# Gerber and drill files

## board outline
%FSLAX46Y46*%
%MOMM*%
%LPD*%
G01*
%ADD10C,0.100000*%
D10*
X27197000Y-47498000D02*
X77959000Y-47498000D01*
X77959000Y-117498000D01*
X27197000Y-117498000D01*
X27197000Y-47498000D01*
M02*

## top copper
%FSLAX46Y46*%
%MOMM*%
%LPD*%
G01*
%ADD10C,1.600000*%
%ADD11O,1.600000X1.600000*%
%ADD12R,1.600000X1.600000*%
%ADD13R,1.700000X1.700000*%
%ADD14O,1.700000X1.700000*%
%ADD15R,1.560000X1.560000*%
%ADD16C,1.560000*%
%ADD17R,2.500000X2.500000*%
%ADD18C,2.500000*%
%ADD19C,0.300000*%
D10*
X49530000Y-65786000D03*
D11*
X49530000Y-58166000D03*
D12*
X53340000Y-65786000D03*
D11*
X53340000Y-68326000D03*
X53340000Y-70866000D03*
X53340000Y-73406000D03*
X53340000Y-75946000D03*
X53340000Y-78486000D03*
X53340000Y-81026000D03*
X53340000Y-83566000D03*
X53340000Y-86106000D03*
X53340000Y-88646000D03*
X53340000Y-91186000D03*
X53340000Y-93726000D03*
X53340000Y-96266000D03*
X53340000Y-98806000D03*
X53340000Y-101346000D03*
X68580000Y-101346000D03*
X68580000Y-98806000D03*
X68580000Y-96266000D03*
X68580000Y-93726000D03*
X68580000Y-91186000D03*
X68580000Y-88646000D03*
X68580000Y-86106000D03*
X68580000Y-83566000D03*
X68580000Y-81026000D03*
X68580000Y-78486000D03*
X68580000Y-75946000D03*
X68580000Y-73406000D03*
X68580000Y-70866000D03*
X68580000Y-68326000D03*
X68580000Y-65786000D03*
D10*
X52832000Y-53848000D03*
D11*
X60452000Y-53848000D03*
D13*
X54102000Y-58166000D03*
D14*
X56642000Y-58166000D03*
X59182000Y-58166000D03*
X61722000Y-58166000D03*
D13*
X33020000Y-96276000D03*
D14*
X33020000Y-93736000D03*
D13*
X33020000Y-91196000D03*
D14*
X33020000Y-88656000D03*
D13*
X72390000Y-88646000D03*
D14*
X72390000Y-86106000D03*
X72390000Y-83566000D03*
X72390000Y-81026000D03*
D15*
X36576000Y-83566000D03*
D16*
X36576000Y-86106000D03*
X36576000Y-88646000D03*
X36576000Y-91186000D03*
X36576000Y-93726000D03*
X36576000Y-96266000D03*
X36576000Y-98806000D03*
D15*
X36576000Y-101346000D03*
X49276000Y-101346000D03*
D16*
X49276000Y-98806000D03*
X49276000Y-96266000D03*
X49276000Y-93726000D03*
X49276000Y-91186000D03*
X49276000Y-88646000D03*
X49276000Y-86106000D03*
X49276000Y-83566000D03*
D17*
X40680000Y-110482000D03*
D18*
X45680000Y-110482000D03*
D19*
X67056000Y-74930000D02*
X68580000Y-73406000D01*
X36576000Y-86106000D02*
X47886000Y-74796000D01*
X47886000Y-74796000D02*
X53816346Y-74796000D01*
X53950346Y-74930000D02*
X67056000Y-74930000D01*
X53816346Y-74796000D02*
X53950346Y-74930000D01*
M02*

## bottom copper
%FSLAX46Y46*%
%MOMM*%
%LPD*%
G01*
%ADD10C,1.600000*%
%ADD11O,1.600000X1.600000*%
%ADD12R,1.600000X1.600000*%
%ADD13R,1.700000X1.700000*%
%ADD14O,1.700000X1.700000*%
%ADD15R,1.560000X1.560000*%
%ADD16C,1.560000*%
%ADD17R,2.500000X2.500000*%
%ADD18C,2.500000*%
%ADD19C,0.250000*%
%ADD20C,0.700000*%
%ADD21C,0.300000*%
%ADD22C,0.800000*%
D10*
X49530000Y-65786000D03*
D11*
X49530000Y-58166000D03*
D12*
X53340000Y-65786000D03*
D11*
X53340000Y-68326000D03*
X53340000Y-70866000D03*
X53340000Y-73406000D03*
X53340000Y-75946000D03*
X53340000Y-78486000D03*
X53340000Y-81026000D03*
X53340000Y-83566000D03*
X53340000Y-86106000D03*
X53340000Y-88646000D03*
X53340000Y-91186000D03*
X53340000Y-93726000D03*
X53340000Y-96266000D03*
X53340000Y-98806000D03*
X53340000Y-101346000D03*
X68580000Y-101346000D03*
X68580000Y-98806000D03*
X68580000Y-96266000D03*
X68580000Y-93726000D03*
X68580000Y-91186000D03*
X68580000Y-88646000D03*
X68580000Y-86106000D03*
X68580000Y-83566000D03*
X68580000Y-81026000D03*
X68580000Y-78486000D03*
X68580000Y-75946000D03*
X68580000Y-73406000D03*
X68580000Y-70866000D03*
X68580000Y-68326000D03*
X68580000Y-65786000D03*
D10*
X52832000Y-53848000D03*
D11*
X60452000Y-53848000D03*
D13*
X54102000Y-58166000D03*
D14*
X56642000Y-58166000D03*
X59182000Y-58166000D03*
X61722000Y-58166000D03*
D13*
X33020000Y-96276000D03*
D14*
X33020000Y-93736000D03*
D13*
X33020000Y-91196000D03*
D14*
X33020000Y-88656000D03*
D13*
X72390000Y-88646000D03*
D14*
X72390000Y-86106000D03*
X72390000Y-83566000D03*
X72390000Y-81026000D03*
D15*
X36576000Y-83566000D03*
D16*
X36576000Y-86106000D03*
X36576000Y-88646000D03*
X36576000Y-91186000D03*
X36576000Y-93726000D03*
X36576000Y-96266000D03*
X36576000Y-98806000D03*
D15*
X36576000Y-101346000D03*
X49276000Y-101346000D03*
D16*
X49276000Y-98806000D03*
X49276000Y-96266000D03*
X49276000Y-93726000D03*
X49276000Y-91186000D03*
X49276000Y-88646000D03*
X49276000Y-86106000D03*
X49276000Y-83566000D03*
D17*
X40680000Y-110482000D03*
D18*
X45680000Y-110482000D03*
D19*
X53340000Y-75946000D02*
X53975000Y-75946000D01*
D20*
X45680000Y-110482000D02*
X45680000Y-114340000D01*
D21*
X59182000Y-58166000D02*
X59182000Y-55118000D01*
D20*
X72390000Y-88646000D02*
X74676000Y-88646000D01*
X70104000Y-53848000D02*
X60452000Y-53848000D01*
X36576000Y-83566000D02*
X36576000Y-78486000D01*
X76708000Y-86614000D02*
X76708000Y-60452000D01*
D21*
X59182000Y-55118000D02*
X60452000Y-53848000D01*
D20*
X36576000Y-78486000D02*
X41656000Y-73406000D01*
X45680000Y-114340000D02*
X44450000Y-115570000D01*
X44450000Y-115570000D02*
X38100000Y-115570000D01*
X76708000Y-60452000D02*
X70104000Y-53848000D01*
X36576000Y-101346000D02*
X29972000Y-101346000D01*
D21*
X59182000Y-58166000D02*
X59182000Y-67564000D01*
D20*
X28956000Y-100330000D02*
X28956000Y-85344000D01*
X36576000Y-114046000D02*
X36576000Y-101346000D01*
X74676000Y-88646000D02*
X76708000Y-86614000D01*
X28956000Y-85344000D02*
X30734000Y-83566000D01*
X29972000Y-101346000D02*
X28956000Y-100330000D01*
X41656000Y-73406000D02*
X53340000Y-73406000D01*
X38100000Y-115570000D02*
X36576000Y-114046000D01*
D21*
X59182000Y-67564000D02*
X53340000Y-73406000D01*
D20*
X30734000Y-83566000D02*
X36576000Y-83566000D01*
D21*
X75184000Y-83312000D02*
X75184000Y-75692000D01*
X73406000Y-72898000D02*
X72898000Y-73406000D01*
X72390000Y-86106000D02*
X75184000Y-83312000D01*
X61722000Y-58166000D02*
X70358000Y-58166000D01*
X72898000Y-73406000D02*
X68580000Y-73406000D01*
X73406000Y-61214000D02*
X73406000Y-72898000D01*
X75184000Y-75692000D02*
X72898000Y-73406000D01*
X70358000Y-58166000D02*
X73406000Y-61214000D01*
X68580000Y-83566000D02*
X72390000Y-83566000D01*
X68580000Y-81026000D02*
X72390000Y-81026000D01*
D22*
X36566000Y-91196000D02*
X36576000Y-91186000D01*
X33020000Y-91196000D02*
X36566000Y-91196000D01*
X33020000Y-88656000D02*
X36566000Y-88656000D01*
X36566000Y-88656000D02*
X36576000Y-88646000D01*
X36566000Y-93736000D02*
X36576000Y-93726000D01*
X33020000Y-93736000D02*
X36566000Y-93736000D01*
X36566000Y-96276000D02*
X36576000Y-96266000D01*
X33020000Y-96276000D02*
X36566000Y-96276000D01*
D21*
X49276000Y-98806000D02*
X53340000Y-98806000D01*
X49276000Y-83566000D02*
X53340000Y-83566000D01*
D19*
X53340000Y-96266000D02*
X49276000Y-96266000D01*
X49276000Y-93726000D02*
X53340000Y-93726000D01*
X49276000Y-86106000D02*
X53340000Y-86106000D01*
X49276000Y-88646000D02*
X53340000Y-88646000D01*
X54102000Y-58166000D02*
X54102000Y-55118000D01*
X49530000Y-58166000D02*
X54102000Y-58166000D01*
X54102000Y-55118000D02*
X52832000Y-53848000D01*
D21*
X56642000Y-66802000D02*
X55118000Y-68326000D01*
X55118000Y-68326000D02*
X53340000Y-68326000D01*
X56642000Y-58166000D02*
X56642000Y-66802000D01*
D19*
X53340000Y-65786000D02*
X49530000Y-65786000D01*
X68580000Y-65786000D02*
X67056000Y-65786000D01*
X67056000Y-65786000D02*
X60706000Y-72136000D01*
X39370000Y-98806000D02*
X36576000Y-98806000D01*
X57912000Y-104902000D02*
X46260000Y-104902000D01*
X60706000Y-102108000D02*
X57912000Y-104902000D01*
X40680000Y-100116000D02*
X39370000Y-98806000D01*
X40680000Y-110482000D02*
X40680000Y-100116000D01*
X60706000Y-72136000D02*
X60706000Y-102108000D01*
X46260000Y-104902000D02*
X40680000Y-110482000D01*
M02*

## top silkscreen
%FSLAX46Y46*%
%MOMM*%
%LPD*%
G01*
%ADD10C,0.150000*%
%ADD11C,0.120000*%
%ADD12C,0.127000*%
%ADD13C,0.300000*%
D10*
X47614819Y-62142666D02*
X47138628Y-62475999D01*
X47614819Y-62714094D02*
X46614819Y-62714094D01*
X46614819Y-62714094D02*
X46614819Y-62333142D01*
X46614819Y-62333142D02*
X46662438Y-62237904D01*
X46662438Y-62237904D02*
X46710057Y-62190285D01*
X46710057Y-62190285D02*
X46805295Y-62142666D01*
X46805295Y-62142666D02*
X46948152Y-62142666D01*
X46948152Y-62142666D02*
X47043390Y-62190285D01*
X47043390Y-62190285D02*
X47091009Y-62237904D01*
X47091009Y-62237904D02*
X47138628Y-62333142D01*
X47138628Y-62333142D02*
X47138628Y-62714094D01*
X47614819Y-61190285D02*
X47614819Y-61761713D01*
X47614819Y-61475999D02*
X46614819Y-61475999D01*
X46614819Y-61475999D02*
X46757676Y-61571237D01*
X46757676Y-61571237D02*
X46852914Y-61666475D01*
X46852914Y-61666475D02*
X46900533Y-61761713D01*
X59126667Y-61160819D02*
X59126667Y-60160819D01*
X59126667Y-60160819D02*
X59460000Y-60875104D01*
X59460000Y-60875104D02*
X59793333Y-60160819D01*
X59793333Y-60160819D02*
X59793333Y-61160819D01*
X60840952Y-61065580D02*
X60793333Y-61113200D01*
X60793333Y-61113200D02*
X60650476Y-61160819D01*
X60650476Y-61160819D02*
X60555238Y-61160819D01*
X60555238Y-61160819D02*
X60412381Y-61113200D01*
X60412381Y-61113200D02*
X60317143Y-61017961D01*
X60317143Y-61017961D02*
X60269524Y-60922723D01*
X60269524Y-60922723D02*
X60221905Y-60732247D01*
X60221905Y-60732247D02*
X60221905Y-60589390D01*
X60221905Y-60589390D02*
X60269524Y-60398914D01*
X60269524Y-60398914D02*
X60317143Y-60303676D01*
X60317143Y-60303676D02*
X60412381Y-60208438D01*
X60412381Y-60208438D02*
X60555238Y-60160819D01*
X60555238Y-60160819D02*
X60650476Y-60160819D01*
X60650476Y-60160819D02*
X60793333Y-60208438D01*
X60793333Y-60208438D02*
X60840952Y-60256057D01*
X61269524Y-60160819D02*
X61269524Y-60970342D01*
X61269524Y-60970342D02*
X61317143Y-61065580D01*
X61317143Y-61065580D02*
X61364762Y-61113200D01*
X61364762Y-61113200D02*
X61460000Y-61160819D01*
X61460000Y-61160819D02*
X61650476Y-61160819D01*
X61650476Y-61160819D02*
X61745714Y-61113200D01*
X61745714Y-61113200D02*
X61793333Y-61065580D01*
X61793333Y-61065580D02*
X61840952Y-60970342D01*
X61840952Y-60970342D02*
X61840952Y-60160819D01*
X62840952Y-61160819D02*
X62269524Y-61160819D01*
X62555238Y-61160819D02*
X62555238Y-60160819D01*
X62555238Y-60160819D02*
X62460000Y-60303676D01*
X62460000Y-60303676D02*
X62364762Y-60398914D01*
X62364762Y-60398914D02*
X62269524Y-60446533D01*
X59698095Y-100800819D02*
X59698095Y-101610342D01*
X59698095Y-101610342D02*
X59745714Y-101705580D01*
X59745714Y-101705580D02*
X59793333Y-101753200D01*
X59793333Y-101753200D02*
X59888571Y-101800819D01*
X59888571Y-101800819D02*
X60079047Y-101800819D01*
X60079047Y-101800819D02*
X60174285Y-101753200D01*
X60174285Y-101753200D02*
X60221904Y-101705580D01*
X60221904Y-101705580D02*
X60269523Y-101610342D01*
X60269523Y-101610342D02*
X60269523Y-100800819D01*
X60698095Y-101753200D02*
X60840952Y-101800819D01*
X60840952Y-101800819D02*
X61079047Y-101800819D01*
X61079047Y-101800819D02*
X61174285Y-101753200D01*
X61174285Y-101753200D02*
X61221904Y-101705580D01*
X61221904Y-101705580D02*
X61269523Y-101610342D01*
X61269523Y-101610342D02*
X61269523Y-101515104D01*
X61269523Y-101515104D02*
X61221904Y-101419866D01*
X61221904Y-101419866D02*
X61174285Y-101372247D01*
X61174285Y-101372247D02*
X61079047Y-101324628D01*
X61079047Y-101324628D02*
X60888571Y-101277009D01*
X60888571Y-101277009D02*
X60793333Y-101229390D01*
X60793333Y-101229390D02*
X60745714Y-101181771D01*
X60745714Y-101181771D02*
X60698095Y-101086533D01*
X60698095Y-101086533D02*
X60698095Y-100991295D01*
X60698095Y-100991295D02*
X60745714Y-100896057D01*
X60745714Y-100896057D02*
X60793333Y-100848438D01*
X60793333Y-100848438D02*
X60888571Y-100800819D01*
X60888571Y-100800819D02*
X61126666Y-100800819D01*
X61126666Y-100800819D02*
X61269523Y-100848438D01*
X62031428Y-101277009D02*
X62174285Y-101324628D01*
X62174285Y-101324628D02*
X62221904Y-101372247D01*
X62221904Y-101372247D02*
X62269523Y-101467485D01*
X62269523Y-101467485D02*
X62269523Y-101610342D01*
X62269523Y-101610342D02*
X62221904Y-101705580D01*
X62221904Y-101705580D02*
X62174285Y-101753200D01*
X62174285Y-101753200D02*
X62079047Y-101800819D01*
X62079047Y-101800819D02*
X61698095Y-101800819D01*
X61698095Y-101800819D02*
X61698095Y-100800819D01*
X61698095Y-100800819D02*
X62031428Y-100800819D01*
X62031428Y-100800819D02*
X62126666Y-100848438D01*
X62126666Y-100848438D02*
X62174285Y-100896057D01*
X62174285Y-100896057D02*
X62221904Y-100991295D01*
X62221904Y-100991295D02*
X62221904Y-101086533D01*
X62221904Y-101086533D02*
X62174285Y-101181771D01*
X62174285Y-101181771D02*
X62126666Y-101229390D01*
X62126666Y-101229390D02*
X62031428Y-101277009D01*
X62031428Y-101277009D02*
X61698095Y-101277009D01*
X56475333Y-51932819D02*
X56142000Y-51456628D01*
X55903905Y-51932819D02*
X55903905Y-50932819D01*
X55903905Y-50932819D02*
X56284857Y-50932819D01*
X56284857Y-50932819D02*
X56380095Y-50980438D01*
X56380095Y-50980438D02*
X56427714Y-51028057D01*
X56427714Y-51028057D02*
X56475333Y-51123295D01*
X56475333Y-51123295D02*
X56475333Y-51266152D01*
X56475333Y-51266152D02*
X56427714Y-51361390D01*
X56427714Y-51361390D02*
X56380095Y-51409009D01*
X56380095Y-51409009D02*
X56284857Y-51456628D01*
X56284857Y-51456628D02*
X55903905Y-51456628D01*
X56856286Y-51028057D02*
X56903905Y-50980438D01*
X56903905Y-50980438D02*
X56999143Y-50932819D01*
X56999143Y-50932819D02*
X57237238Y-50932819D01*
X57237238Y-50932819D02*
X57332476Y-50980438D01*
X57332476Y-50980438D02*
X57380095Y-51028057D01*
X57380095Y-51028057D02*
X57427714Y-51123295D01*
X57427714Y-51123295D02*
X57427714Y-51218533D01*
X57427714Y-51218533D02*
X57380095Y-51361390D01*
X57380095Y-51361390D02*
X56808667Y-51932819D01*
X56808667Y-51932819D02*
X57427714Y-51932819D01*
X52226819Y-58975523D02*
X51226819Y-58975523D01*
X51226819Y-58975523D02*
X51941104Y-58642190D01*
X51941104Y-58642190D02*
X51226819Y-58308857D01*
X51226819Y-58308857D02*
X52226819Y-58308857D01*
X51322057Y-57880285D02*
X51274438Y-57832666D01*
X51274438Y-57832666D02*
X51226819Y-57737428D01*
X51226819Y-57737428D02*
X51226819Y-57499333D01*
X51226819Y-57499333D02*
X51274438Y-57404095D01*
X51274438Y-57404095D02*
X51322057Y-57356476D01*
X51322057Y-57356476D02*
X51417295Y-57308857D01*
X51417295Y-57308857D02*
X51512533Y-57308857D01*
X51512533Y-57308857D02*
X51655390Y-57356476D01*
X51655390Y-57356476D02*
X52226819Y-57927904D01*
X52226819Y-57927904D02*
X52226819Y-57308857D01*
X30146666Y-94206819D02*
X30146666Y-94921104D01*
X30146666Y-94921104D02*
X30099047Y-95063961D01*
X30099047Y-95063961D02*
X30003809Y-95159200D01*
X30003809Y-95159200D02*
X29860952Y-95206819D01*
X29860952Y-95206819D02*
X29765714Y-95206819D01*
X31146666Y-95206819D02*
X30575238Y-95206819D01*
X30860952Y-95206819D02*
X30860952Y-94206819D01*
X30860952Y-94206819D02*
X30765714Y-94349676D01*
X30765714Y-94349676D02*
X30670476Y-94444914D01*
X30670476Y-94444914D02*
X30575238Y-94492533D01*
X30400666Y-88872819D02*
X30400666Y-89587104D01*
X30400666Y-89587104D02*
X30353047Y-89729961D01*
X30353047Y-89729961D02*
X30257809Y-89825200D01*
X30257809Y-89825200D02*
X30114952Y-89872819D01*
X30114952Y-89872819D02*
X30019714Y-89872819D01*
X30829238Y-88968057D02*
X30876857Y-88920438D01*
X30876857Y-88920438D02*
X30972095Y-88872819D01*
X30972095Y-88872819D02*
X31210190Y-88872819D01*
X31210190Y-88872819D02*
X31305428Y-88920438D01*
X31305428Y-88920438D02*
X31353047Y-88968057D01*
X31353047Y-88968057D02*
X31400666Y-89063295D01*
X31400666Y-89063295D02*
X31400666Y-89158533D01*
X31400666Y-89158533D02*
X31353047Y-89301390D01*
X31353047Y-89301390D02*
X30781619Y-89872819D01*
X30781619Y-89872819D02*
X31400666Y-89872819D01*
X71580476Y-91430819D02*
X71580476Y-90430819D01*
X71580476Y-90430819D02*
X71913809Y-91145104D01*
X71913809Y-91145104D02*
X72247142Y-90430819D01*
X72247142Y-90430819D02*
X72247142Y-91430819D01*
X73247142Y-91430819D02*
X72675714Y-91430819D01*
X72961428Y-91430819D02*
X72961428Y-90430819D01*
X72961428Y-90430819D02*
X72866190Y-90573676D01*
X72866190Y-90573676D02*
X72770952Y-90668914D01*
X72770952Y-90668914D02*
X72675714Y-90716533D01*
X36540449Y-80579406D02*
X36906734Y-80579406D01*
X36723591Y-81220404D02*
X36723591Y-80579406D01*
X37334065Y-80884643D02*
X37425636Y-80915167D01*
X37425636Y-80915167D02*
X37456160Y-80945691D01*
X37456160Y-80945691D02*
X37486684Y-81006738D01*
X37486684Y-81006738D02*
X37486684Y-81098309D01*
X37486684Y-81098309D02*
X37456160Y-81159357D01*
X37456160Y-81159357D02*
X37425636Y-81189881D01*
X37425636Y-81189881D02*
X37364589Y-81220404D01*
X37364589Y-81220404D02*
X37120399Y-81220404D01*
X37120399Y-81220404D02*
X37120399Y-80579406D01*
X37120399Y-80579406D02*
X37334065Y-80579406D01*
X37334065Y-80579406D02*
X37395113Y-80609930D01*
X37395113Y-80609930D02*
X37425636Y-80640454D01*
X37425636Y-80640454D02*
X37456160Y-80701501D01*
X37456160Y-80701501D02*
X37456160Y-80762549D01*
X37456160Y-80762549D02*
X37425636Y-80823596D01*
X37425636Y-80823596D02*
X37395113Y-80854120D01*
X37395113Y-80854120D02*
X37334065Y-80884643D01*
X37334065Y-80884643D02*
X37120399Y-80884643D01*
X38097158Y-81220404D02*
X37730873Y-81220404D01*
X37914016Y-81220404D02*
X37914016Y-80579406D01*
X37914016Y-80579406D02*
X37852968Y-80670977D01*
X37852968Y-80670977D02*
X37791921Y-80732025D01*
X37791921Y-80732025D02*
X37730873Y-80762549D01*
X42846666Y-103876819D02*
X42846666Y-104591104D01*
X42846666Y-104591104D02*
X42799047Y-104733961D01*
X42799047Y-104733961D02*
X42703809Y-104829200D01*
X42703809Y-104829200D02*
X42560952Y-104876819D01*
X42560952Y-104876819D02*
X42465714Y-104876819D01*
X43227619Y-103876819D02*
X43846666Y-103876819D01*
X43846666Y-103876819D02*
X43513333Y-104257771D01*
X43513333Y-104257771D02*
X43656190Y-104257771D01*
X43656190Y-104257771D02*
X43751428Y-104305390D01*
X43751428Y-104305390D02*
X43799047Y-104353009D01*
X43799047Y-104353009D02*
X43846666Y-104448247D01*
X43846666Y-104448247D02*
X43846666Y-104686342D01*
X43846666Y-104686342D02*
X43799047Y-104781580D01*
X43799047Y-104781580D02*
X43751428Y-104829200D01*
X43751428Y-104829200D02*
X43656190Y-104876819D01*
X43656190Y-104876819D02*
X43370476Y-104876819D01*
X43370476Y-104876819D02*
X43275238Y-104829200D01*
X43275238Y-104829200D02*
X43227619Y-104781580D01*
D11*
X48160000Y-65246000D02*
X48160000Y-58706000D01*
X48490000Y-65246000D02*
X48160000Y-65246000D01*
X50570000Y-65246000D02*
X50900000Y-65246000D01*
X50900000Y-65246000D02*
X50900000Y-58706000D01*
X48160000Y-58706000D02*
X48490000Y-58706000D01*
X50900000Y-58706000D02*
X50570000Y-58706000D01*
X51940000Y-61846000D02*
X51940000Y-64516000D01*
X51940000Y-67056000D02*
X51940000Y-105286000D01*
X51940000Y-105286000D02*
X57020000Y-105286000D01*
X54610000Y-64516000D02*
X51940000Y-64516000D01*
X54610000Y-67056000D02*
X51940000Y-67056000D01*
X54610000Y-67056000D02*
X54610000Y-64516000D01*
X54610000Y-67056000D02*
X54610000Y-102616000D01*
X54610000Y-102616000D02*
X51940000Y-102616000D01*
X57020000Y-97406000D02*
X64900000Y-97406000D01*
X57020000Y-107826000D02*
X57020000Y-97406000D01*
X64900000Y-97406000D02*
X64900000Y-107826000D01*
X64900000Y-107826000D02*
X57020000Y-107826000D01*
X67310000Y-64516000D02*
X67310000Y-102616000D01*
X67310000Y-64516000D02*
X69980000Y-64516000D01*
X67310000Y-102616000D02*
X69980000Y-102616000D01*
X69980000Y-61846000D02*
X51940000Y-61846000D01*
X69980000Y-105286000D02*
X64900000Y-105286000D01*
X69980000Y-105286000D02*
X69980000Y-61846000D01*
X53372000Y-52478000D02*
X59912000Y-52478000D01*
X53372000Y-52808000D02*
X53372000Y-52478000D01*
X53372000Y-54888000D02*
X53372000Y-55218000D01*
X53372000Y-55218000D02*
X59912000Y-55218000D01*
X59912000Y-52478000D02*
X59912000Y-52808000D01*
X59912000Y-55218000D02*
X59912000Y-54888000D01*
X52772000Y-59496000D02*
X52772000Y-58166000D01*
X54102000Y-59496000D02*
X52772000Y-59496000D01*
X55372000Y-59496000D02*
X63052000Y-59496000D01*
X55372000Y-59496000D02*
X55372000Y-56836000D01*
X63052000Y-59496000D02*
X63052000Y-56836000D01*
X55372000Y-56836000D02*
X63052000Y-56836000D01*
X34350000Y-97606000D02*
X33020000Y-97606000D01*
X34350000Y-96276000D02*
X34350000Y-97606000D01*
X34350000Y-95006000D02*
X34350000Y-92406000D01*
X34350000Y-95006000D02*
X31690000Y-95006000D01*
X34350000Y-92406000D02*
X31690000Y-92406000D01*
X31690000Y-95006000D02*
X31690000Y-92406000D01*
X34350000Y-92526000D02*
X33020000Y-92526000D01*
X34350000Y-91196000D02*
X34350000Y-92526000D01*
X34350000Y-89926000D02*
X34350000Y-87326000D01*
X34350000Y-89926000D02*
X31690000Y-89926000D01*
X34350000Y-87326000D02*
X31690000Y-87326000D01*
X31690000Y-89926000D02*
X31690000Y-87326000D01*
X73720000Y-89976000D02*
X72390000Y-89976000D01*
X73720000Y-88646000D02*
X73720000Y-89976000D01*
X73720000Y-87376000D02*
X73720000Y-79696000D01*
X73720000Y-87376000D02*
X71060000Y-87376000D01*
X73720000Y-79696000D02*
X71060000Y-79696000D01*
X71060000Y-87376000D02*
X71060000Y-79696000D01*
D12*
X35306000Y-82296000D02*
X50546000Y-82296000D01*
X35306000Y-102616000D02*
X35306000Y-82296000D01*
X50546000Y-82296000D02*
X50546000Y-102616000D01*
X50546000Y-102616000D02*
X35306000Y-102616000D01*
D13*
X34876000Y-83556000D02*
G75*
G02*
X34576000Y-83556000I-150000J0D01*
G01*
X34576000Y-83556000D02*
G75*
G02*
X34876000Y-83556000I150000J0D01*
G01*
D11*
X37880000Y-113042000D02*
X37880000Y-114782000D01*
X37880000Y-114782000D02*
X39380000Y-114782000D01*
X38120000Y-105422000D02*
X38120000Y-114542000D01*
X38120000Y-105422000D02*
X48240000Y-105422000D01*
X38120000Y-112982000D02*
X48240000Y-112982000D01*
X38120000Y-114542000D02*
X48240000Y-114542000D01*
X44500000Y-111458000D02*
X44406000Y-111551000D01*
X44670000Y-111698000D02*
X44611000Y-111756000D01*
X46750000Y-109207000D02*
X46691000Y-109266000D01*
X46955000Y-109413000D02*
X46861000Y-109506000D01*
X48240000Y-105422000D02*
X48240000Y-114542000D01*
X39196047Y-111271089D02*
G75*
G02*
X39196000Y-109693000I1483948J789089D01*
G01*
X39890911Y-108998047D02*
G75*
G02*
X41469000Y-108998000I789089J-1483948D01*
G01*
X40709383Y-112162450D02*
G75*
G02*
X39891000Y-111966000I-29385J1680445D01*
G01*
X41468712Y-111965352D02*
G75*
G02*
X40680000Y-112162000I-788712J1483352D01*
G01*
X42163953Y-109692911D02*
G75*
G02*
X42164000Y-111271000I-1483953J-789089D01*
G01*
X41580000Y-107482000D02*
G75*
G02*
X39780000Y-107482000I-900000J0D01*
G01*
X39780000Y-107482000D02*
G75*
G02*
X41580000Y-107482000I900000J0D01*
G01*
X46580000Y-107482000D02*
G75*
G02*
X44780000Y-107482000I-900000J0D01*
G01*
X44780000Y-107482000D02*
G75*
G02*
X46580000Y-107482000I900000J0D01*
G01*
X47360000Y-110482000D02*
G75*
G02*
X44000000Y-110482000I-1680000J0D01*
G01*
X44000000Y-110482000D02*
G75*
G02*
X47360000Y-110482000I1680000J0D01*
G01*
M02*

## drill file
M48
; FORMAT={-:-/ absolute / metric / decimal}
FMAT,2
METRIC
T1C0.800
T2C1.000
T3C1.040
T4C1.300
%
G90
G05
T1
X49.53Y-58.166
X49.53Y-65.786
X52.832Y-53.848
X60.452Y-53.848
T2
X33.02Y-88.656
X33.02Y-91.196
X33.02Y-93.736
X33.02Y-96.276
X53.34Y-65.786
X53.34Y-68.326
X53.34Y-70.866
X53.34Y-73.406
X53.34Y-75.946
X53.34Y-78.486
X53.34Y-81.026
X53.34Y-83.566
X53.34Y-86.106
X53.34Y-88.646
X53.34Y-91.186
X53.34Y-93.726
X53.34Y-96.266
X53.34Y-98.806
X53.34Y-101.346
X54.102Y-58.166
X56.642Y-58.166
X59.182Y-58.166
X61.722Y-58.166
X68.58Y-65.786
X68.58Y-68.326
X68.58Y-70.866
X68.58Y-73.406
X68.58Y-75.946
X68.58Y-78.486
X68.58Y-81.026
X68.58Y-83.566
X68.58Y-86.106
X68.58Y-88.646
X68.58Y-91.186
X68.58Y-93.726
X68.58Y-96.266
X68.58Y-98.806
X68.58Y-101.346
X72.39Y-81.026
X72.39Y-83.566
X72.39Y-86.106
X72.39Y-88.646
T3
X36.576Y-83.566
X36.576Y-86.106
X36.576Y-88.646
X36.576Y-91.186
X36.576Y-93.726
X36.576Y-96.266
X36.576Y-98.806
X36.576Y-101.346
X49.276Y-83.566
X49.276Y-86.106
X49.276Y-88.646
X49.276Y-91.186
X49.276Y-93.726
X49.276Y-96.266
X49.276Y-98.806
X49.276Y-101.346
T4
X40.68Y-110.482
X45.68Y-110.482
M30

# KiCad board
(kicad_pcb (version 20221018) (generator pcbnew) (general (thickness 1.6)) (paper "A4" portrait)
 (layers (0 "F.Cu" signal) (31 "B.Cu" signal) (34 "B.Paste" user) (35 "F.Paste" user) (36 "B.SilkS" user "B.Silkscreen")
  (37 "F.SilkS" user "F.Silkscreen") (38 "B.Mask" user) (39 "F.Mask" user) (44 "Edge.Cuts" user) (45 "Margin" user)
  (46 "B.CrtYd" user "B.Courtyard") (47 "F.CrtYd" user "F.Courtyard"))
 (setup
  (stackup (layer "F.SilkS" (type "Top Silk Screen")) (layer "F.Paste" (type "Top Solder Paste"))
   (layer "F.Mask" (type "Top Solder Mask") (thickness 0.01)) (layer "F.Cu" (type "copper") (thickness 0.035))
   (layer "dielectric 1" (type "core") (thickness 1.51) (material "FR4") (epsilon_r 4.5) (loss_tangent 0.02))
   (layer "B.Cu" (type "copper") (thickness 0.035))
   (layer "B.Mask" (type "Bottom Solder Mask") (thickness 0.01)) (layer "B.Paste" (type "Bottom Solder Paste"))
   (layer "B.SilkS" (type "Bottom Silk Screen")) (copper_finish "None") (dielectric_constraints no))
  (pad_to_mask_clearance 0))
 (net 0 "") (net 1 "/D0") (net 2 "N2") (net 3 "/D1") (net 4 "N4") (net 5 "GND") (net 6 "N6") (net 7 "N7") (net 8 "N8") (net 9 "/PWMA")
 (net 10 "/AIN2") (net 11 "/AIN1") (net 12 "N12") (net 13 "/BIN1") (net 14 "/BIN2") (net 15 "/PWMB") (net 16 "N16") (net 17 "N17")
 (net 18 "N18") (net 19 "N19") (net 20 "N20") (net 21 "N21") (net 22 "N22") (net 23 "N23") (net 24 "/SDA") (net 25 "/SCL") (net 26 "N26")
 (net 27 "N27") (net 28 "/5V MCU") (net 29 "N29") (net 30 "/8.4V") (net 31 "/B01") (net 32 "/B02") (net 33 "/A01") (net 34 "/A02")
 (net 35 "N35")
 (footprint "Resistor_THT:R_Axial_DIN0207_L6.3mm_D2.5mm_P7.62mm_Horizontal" (layer "F.Cu") (at 49.53 65.786 90)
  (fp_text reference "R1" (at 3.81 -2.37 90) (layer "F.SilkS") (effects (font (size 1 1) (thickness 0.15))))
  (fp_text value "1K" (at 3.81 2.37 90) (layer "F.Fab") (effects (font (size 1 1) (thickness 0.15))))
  (fp_line (start 0.54 -1.37) (end 7.08 -1.37) (stroke (width 0.12) (type solid)) (layer "F.SilkS"))
  (fp_line (start 0.54 -1.04) (end 0.54 -1.37) (stroke (width 0.12) (type solid)) (layer "F.SilkS"))
  (fp_line (start 0.54 1.04) (end 0.54 1.37) (stroke (width 0.12) (type solid)) (layer "F.SilkS"))
  (fp_line (start 0.54 1.37) (end 7.08 1.37) (stroke (width 0.12) (type solid)) (layer "F.SilkS"))
  (fp_line (start 7.08 -1.37) (end 7.08 -1.04) (stroke (width 0.12) (type solid)) (layer "F.SilkS"))
  (fp_line (start 7.08 1.37) (end 7.08 1.04) (stroke (width 0.12) (type solid)) (layer "F.SilkS"))
  (pad "1" thru_hole circle (at 0 0 90) (size 1.6 1.6) (drill 0.8) (layers "*.Cu" "*.Mask") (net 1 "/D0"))
  (pad "2" thru_hole oval (at 7.62 0 90) (size 1.6 1.6) (drill 0.8) (layers "*.Cu" "*.Mask") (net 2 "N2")))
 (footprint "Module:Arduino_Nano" (layer "F.Cu") (at 53.34 65.786)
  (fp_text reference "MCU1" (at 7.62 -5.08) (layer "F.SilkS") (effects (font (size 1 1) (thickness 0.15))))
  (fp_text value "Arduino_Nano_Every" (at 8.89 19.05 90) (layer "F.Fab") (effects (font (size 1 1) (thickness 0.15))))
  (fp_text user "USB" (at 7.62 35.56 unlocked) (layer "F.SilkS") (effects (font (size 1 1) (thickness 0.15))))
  (fp_line (start -1.4 -3.94) (end -1.4 -1.27) (stroke (width 0.12) (type solid)) (layer "F.SilkS"))
  (fp_line (start -1.4 1.27) (end -1.4 39.5) (stroke (width 0.12) (type solid)) (layer "F.SilkS"))
  (fp_line (start -1.4 39.5) (end 3.68 39.5) (stroke (width 0.12) (type solid)) (layer "F.SilkS"))
  (fp_line (start 1.27 -1.27) (end -1.4 -1.27) (stroke (width 0.12) (type solid)) (layer "F.SilkS"))
  (fp_line (start 1.27 1.27) (end -1.4 1.27) (stroke (width 0.12) (type solid)) (layer "F.SilkS"))
  (fp_line (start 1.27 1.27) (end 1.27 -1.27) (stroke (width 0.12) (type solid)) (layer "F.SilkS"))
  (fp_line (start 1.27 1.27) (end 1.27 36.83) (stroke (width 0.12) (type solid)) (layer "F.SilkS"))
  (fp_line (start 1.27 36.83) (end -1.4 36.83) (stroke (width 0.12) (type solid)) (layer "F.SilkS"))
  (fp_line (start 3.68 31.62) (end 11.56 31.62) (stroke (width 0.12) (type solid)) (layer "F.SilkS"))
  (fp_line (start 3.68 42.04) (end 3.68 31.62) (stroke (width 0.12) (type solid)) (layer "F.SilkS"))
  (fp_line (start 11.56 31.62) (end 11.56 42.04) (stroke (width 0.12) (type solid)) (layer "F.SilkS"))
  (fp_line (start 11.56 42.04) (end 3.68 42.04) (stroke (width 0.12) (type solid)) (layer "F.SilkS"))
  (fp_line (start 13.97 -1.27) (end 13.97 36.83) (stroke (width 0.12) (type solid)) (layer "F.SilkS"))
  (fp_line (start 13.97 -1.27) (end 16.64 -1.27) (stroke (width 0.12) (type solid)) (layer "F.SilkS"))
  (fp_line (start 13.97 36.83) (end 16.64 36.83) (stroke (width 0.12) (type solid)) (layer "F.SilkS"))
  (fp_line (start 16.64 -3.94) (end -1.4 -3.94) (stroke (width 0.12) (type solid)) (layer "F.SilkS"))
  (fp_line (start 16.64 39.5) (end 11.56 39.5) (stroke (width 0.12) (type solid)) (layer "F.SilkS"))
  (fp_line (start 16.64 39.5) (end 16.64 -3.94) (stroke (width 0.12) (type solid)) (layer "F.SilkS"))
  (pad "1" thru_hole rect (at 0 0) (size 1.6 1.6) (drill 1) (layers "*.Cu" "*.Mask") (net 1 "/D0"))
  (pad "2" thru_hole oval (at 0 2.54) (size 1.6 1.6) (drill 1) (layers "*.Cu" "*.Mask") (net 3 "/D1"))
  (pad "3" thru_hole oval (at 0 5.08) (size 1.6 1.6) (drill 1) (layers "*.Cu" "*.Mask") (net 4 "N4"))
  (pad "4" thru_hole oval (at 0 7.62) (size 1.6 1.6) (drill 1) (layers "*.Cu" "*.Mask") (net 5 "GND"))
  (pad "5" thru_hole oval (at 0 10.16) (size 1.6 1.6) (drill 1) (layers "*.Cu" "*.Mask") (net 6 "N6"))
  (pad "6" thru_hole oval (at 0 12.7) (size 1.6 1.6) (drill 1) (layers "*.Cu" "*.Mask") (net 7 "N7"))
  (pad "7" thru_hole oval (at 0 15.24) (size 1.6 1.6) (drill 1) (layers "*.Cu" "*.Mask") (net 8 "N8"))
  (pad "8" thru_hole oval (at 0 17.78) (size 1.6 1.6) (drill 1) (layers "*.Cu" "*.Mask") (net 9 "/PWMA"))
  (pad "9" thru_hole oval (at 0 20.32) (size 1.6 1.6) (drill 1) (layers "*.Cu" "*.Mask") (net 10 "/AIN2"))
  (pad "10" thru_hole oval (at 0 22.86) (size 1.6 1.6) (drill 1) (layers "*.Cu" "*.Mask") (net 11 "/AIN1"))
  (pad "11" thru_hole oval (at 0 25.4) (size 1.6 1.6) (drill 1) (layers "*.Cu" "*.Mask") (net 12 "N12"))
  (pad "12" thru_hole oval (at 0 27.94) (size 1.6 1.6) (drill 1) (layers "*.Cu" "*.Mask") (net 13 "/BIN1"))
  (pad "13" thru_hole oval (at 0 30.48) (size 1.6 1.6) (drill 1) (layers "*.Cu" "*.Mask") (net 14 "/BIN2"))
  (pad "14" thru_hole oval (at 0 33.02) (size 1.6 1.6) (drill 1) (layers "*.Cu" "*.Mask") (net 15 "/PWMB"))
  (pad "15" thru_hole oval (at 0 35.56) (size 1.6 1.6) (drill 1) (layers "*.Cu" "*.Mask") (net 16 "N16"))
  (pad "16" thru_hole oval (at 15.24 35.56) (size 1.6 1.6) (drill 1) (layers "*.Cu" "*.Mask") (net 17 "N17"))
  (pad "17" thru_hole oval (at 15.24 33.02) (size 1.6 1.6) (drill 1) (layers "*.Cu" "*.Mask") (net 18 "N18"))
  (pad "18" thru_hole oval (at 15.24 30.48) (size 1.6 1.6) (drill 1) (layers "*.Cu" "*.Mask") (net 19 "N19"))
  (pad "19" thru_hole oval (at 15.24 27.94) (size 1.6 1.6) (drill 1) (layers "*.Cu" "*.Mask") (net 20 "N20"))
  (pad "20" thru_hole oval (at 15.24 25.4) (size 1.6 1.6) (drill 1) (layers "*.Cu" "*.Mask") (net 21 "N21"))
  (pad "21" thru_hole oval (at 15.24 22.86) (size 1.6 1.6) (drill 1) (layers "*.Cu" "*.Mask") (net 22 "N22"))
  (pad "22" thru_hole oval (at 15.24 20.32) (size 1.6 1.6) (drill 1) (layers "*.Cu" "*.Mask") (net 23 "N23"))
  (pad "23" thru_hole oval (at 15.24 17.78) (size 1.6 1.6) (drill 1) (layers "*.Cu" "*.Mask") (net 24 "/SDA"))
  (pad "24" thru_hole oval (at 15.24 15.24) (size 1.6 1.6) (drill 1) (layers "*.Cu" "*.Mask") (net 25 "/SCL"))
  (pad "25" thru_hole oval (at 15.24 12.7) (size 1.6 1.6) (drill 1) (layers "*.Cu" "*.Mask") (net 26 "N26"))
  (pad "26" thru_hole oval (at 15.24 10.16) (size 1.6 1.6) (drill 1) (layers "*.Cu" "*.Mask") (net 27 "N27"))
  (pad "27" thru_hole oval (at 15.24 7.62) (size 1.6 1.6) (drill 1) (layers "*.Cu" "*.Mask") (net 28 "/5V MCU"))
  (pad "28" thru_hole oval (at 15.24 5.08) (size 1.6 1.6) (drill 1) (layers "*.Cu" "*.Mask") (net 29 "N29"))
  (pad "29" thru_hole oval (at 15.24 2.54) (size 1.6 1.6) (drill 1) (layers "*.Cu" "*.Mask") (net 5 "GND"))
  (pad "30" thru_hole oval (at 15.24 0) (size 1.6 1.6) (drill 1) (layers "*.Cu" "*.Mask") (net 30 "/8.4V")))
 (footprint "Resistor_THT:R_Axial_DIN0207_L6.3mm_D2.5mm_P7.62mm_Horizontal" (layer "F.Cu") (at 52.832 53.848)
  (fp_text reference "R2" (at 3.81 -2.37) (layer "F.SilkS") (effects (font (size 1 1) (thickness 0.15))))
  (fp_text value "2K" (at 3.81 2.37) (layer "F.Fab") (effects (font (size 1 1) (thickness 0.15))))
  (fp_line (start 0.54 -1.37) (end 7.08 -1.37) (stroke (width 0.12) (type solid)) (layer "F.SilkS"))
  (fp_line (start 0.54 -1.04) (end 0.54 -1.37) (stroke (width 0.12) (type solid)) (layer "F.SilkS"))
  (fp_line (start 0.54 1.04) (end 0.54 1.37) (stroke (width 0.12) (type solid)) (layer "F.SilkS"))
  (fp_line (start 0.54 1.37) (end 7.08 1.37) (stroke (width 0.12) (type solid)) (layer "F.SilkS"))
  (fp_line (start 7.08 -1.37) (end 7.08 -1.04) (stroke (width 0.12) (type solid)) (layer "F.SilkS"))
  (fp_line (start 7.08 1.37) (end 7.08 1.04) (stroke (width 0.12) (type solid)) (layer "F.SilkS"))
  (pad "1" thru_hole circle (at 0 0) (size 1.6 1.6) (drill 0.8) (layers "*.Cu" "*.Mask") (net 2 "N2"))
  (pad "2" thru_hole oval (at 7.62 0) (size 1.6 1.6) (drill 0.8) (layers "*.Cu" "*.Mask") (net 5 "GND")))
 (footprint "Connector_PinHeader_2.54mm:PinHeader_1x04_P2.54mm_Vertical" (layer "F.Cu") (at 54.102 58.166 90)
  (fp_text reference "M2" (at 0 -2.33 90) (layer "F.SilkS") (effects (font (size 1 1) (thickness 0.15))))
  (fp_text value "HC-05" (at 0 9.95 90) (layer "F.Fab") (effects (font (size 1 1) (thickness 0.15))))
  (fp_line (start -1.33 -1.33) (end 0 -1.33) (stroke (width 0.12) (type solid)) (layer "F.SilkS"))
  (fp_line (start -1.33 0) (end -1.33 -1.33) (stroke (width 0.12) (type solid)) (layer "F.SilkS"))
  (fp_line (start -1.33 1.27) (end -1.33 8.95) (stroke (width 0.12) (type solid)) (layer "F.SilkS"))
  (fp_line (start -1.33 1.27) (end 1.33 1.27) (stroke (width 0.12) (type solid)) (layer "F.SilkS"))
  (fp_line (start -1.33 8.95) (end 1.33 8.95) (stroke (width 0.12) (type solid)) (layer "F.SilkS"))
  (fp_line (start 1.33 1.27) (end 1.33 8.95) (stroke (width 0.12) (type solid)) (layer "F.SilkS"))
  (pad "1" thru_hole rect (at 0 0 90) (size 1.7 1.7) (drill 1) (layers "*.Cu" "*.Mask") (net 2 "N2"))
  (pad "2" thru_hole oval (at 0 2.54 90) (size 1.7 1.7) (drill 1) (layers "*.Cu" "*.Mask") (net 3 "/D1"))
  (pad "3" thru_hole oval (at 0 5.08 90) (size 1.7 1.7) (drill 1) (layers "*.Cu" "*.Mask") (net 5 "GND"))
  (pad "4" thru_hole oval (at 0 7.62 90) (size 1.7 1.7) (drill 1) (layers "*.Cu" "*.Mask") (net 28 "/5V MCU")))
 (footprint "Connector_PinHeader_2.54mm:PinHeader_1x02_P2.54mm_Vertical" (layer "F.Cu") (at 33.02 96.276 180)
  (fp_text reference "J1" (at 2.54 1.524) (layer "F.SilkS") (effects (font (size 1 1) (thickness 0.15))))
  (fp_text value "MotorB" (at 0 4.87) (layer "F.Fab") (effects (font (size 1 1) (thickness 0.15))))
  (fp_line (start -1.33 -1.33) (end 0 -1.33) (stroke (width 0.12) (type solid)) (layer "F.SilkS"))
  (fp_line (start -1.33 0) (end -1.33 -1.33) (stroke (width 0.12) (type solid)) (layer "F.SilkS"))
  (fp_line (start -1.33 1.27) (end -1.33 3.87) (stroke (width 0.12) (type solid)) (layer "F.SilkS"))
  (fp_line (start -1.33 1.27) (end 1.33 1.27) (stroke (width 0.12) (type solid)) (layer "F.SilkS"))
  (fp_line (start -1.33 3.87) (end 1.33 3.87) (stroke (width 0.12) (type solid)) (layer "F.SilkS"))
  (fp_line (start 1.33 1.27) (end 1.33 3.87) (stroke (width 0.12) (type solid)) (layer "F.SilkS"))
  (pad "1" thru_hole rect (at 0 0 180) (size 1.7 1.7) (drill 1) (layers "*.Cu" "*.Mask") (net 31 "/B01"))
  (pad "2" thru_hole oval (at 0 2.54 180) (size 1.7 1.7) (drill 1) (layers "*.Cu" "*.Mask") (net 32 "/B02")))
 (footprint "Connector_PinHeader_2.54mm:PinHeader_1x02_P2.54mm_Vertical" (layer "F.Cu") (at 33.02 91.196 180)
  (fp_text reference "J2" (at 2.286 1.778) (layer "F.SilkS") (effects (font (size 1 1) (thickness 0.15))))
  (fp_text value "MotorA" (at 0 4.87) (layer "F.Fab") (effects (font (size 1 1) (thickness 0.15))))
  (fp_line (start -1.33 -1.33) (end 0 -1.33) (stroke (width 0.12) (type solid)) (layer "F.SilkS"))
  (fp_line (start -1.33 0) (end -1.33 -1.33) (stroke (width 0.12) (type solid)) (layer "F.SilkS"))
  (fp_line (start -1.33 1.27) (end -1.33 3.87) (stroke (width 0.12) (type solid)) (layer "F.SilkS"))
  (fp_line (start -1.33 1.27) (end 1.33 1.27) (stroke (width 0.12) (type solid)) (layer "F.SilkS"))
  (fp_line (start -1.33 3.87) (end 1.33 3.87) (stroke (width 0.12) (type solid)) (layer "F.SilkS"))
  (fp_line (start 1.33 1.27) (end 1.33 3.87) (stroke (width 0.12) (type solid)) (layer "F.SilkS"))
  (pad "1" thru_hole rect (at 0 0 180) (size 1.7 1.7) (drill 1) (layers "*.Cu" "*.Mask") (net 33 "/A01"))
  (pad "2" thru_hole oval (at 0 2.54 180) (size 1.7 1.7) (drill 1) (layers "*.Cu" "*.Mask") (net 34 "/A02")))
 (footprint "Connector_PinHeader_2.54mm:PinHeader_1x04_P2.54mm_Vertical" (layer "F.Cu") (at 72.39 88.646 180)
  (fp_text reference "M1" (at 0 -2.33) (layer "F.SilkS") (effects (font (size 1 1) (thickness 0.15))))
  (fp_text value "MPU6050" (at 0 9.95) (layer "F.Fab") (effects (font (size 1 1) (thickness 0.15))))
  (fp_line (start -1.33 -1.33) (end 0 -1.33) (stroke (width 0.12) (type solid)) (layer "F.SilkS"))
  (fp_line (start -1.33 0) (end -1.33 -1.33) (stroke (width 0.12) (type solid)) (layer "F.SilkS"))
  (fp_line (start -1.33 1.27) (end -1.33 8.95) (stroke (width 0.12) (type solid)) (layer "F.SilkS"))
  (fp_line (start -1.33 1.27) (end 1.33 1.27) (stroke (width 0.12) (type solid)) (layer "F.SilkS"))
  (fp_line (start -1.33 8.95) (end 1.33 8.95) (stroke (width 0.12) (type solid)) (layer "F.SilkS"))
  (fp_line (start 1.33 1.27) (end 1.33 8.95) (stroke (width 0.12) (type solid)) (layer "F.SilkS"))
  (pad "1" thru_hole rect (at 0 0 180) (size 1.7 1.7) (drill 1) (layers "*.Cu" "*.Mask") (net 5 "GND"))
  (pad "2" thru_hole oval (at 0 2.54 180) (size 1.7 1.7) (drill 1) (layers "*.Cu" "*.Mask") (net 28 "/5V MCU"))
  (pad "3" thru_hole oval (at 0 5.08 180) (size 1.7 1.7) (drill 1) (layers "*.Cu" "*.Mask") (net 24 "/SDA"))
  (pad "4" thru_hole oval (at 0 7.62 180) (size 1.7 1.7) (drill 1) (layers "*.Cu" "*.Mask") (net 25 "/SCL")))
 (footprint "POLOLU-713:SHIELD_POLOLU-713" (layer "F.Cu") (at 42.926 92.456)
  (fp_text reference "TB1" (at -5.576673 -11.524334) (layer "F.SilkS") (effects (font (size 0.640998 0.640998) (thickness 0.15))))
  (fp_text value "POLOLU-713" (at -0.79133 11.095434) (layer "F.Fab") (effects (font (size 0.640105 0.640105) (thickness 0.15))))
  (fp_line (start -7.62 -10.16) (end 7.62 -10.16) (stroke (width 0.127) (type solid)) (layer "F.SilkS"))
  (fp_line (start -7.62 10.16) (end -7.62 -10.16) (stroke (width 0.127) (type solid)) (layer "F.SilkS"))
  (fp_line (start 7.62 -10.16) (end 7.62 10.16) (stroke (width 0.127) (type solid)) (layer "F.SilkS"))
  (fp_line (start 7.62 10.16) (end -7.62 10.16) (stroke (width 0.127) (type solid)) (layer "F.SilkS"))
  (fp_circle (center -8.2 -8.9) (end -8.05 -8.9) (stroke (width 0.3) (type solid)) (fill none) (layer "F.SilkS"))
  (pad "1" thru_hole rect (at -6.35 -8.89) (size 1.56 1.56) (drill 1.04) (layers "*.Cu" "*.Mask") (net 5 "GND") (solder_mask_margin 0.102))
  (pad "2" thru_hole circle (at -6.35 -6.35) (size 1.56 1.56) (drill 1.04) (layers "*.Cu" "*.Mask") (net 28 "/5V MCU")
   (solder_mask_margin 0.102))
  (pad "3" thru_hole circle (at -6.35 -3.81) (size 1.56 1.56) (drill 1.04) (layers "*.Cu" "*.Mask") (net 34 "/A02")
   (solder_mask_margin 0.102))
  (pad "4" thru_hole circle (at -6.35 -1.27) (size 1.56 1.56) (drill 1.04) (layers "*.Cu" "*.Mask") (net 33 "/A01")
   (solder_mask_margin 0.102))
  (pad "5" thru_hole circle (at -6.35 1.27) (size 1.56 1.56) (drill 1.04) (layers "*.Cu" "*.Mask") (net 32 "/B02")
   (solder_mask_margin 0.102))
  (pad "6" thru_hole circle (at -6.35 3.81) (size 1.56 1.56) (drill 1.04) (layers "*.Cu" "*.Mask") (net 31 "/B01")
   (solder_mask_margin 0.102))
  (pad "7" thru_hole circle (at -6.35 6.35) (size 1.56 1.56) (drill 1.04) (layers "*.Cu" "*.Mask") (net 30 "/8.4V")
   (solder_mask_margin 0.102))
  (pad "8" thru_hole rect (at -6.35 8.89) (size 1.56 1.56) (drill 1.04) (layers "*.Cu" "*.Mask") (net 5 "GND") (solder_mask_margin 0.102))
  (pad "9" thru_hole rect (at 6.35 8.89) (size 1.56 1.56) (drill 1.04) (layers "*.Cu" "*.Mask") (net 5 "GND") (solder_mask_margin 0.102))
  (pad "10" thru_hole circle (at 6.35 6.35) (size 1.56 1.56) (drill 1.04) (layers "*.Cu" "*.Mask") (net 15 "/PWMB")
   (solder_mask_margin 0.102))
  (pad "11" thru_hole circle (at 6.35 3.81) (size 1.56 1.56) (drill 1.04) (layers "*.Cu" "*.Mask") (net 14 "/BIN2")
   (solder_mask_margin 0.102))
  (pad "12" thru_hole circle (at 6.35 1.27) (size 1.56 1.56) (drill 1.04) (layers "*.Cu" "*.Mask") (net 13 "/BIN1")
   (solder_mask_margin 0.102))
  (pad "13" thru_hole circle (at 6.35 -1.27) (size 1.56 1.56) (drill 1.04) (layers "*.Cu" "*.Mask") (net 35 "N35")
   (solder_mask_margin 0.102))
  (pad "14" thru_hole circle (at 6.35 -3.81) (size 1.56 1.56) (drill 1.04) (layers "*.Cu" "*.Mask") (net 11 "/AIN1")
   (solder_mask_margin 0.102))
  (pad "15" thru_hole circle (at 6.35 -6.35) (size 1.56 1.56) (drill 1.04) (layers "*.Cu" "*.Mask") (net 10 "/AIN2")
   (solder_mask_margin 0.102))
  (pad "16" thru_hole circle (at 6.35 -8.89) (size 1.56 1.56) (drill 1.04) (layers "*.Cu" "*.Mask") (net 9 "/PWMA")
   (solder_mask_margin 0.102)))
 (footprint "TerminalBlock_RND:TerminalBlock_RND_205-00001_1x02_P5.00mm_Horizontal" (layer "F.Cu") (at 40.68 110.482)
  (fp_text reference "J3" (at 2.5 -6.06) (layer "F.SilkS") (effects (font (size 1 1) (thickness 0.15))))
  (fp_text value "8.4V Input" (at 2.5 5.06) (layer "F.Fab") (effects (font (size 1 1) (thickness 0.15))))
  (fp_line (start -2.8 2.56) (end -2.8 4.3) (stroke (width 0.12) (type solid)) (layer "F.SilkS"))
  (fp_line (start -2.8 4.3) (end -1.3 4.3) (stroke (width 0.12) (type solid)) (layer "F.SilkS"))
  (fp_line (start -2.56 -5.06) (end -2.56 4.06) (stroke (width 0.12) (type solid)) (layer "F.SilkS"))
  (fp_line (start -2.56 -5.06) (end 7.56 -5.06) (stroke (width 0.12) (type solid)) (layer "F.SilkS"))
  (fp_line (start -2.56 2.5) (end 7.56 2.5) (stroke (width 0.12) (type solid)) (layer "F.SilkS"))
  (fp_line (start -2.56 4.06) (end 7.56 4.06) (stroke (width 0.12) (type solid)) (layer "F.SilkS"))
  (fp_line (start 3.82 0.976) (end 3.726 1.069) (stroke (width 0.12) (type solid)) (layer "F.SilkS"))
  (fp_line (start 3.99 1.216) (end 3.931 1.274) (stroke (width 0.12) (type solid)) (layer "F.SilkS"))
  (fp_line (start 6.07 -1.275) (end 6.011 -1.216) (stroke (width 0.12) (type solid)) (layer "F.SilkS"))
  (fp_line (start 6.275 -1.069) (end 6.181 -0.976) (stroke (width 0.12) (type solid)) (layer "F.SilkS"))
  (fp_line (start 7.56 -5.06) (end 7.56 4.06) (stroke (width 0.12) (type solid)) (layer "F.SilkS"))
  (fp_arc (start -1.483953 0.789089) (mid -1.680708 0.00005) (end -1.484 -0.789) (stroke (width 0.12) (type solid)) (layer "F.SilkS"))
  (fp_arc (start -0.789089 -1.483953) (mid -0.00005 -1.680708) (end 0.789 -1.484) (stroke (width 0.12) (type solid)) (layer "F.SilkS"))
  (fp_arc (start 0.029383 1.68045) (mid -0.392304 1.634281) (end -0.789 1.484) (stroke (width 0.12) (type solid)) (layer "F.SilkS"))
  (fp_arc (start 0.788712 1.483352) (mid 0.406429 1.630097) (end 0 1.68) (stroke (width 0.12) (type solid)) (layer "F.SilkS"))
  (fp_arc (start 1.483953 -0.789089) (mid 1.680708 -0.00005) (end 1.484 0.789) (stroke (width 0.12) (type solid)) (layer "F.SilkS"))
  (fp_circle (center 0 -3) (end 0.9 -3) (stroke (width 0.12) (type solid)) (fill none) (layer "F.SilkS"))
  (fp_circle (center 5 -3) (end 5.9 -3) (stroke (width 0.12) (type solid)) (fill none) (layer "F.SilkS"))
  (fp_circle (center 5 0) (end 6.68 0) (stroke (width 0.12) (type solid)) (fill none) (layer "F.SilkS"))
  (pad "1" thru_hole rect (at 0 0) (size 2.5 2.5) (drill 1.3) (layers "*.Cu" "*.Mask") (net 30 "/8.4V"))
  (pad "2" thru_hole circle (at 5 0) (size 2.5 2.5) (drill 1.3) (layers "*.Cu" "*.Mask") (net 5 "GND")))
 (gr_rect (start 27.197 47.498) (end 77.959 117.498) (stroke (width 0.1) (type default)) (fill none) (layer "Edge.Cuts"))
 (segment (start 53.34 75.946) (end 53.975 75.946) (width 0.25) (layer "B.Cu") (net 6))
 (segment (start 45.68 110.482) (end 45.68 114.34) (width 0.7) (layer "B.Cu") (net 5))
 (segment (start 59.182 58.166) (end 59.182 55.118) (width 0.3) (layer "B.Cu") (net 5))
 (segment (start 72.39 88.646) (end 74.676 88.646) (width 0.7) (layer "B.Cu") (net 5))
 (segment (start 70.104 53.848) (end 60.452 53.848) (width 0.7) (layer "B.Cu") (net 5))
 (segment (start 36.576 83.566) (end 36.576 78.486) (width 0.7) (layer "B.Cu") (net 5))
 (segment (start 76.708 86.614) (end 76.708 60.452) (width 0.7) (layer "B.Cu") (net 5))
 (segment (start 59.182 55.118) (end 60.452 53.848) (width 0.3) (layer "B.Cu") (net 5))
 (segment (start 36.576 78.486) (end 41.656 73.406) (width 0.7) (layer "B.Cu") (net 5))
 (segment (start 45.68 114.34) (end 44.45 115.57) (width 0.7) (layer "B.Cu") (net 5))
 (segment (start 44.45 115.57) (end 38.1 115.57) (width 0.7) (layer "B.Cu") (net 5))
 (segment (start 76.708 60.452) (end 70.104 53.848) (width 0.7) (layer "B.Cu") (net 5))
 (segment (start 36.576 101.346) (end 29.972 101.346) (width 0.7) (layer "B.Cu") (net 5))
 (segment (start 59.182 58.166) (end 59.182 67.564) (width 0.3) (layer "B.Cu") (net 5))
 (segment (start 28.956 100.33) (end 28.956 85.344) (width 0.7) (layer "B.Cu") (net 5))
 (segment (start 36.576 114.046) (end 36.576 101.346) (width 0.7) (layer "B.Cu") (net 5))
 (segment (start 74.676 88.646) (end 76.708 86.614) (width 0.7) (layer "B.Cu") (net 5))
 (segment (start 28.956 85.344) (end 30.734 83.566) (width 0.7) (layer "B.Cu") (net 5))
 (segment (start 29.972 101.346) (end 28.956 100.33) (width 0.7) (layer "B.Cu") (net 5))
 (segment (start 41.656 73.406) (end 53.34 73.406) (width 0.7) (layer "B.Cu") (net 5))
 (segment (start 38.1 115.57) (end 36.576 114.046) (width 0.7) (layer "B.Cu") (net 5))
 (segment (start 59.182 67.564) (end 53.34 73.406) (width 0.3) (layer "B.Cu") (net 5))
 (segment (start 30.734 83.566) (end 36.576 83.566) (width 0.7) (layer "B.Cu") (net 5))
 (segment (start 67.056 74.93) (end 68.58 73.406) (width 0.3) (layer "F.Cu") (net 28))
 (segment (start 36.576 86.106) (end 47.886 74.796) (width 0.3) (layer "F.Cu") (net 28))
 (segment (start 47.886 74.796) (end 53.816346 74.796) (width 0.3) (layer "F.Cu") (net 28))
 (segment (start 53.950346 74.93) (end 67.056 74.93) (width 0.3) (layer "F.Cu") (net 28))
 (segment (start 53.816346 74.796) (end 53.950346 74.93) (width 0.3) (layer "F.Cu") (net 28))
 (segment (start 75.184 83.312) (end 75.184 75.692) (width 0.3) (layer "B.Cu") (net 28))
 (segment (start 73.406 72.898) (end 72.898 73.406) (width 0.3) (layer "B.Cu") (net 28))
 (segment (start 72.39 86.106) (end 75.184 83.312) (width 0.3) (layer "B.Cu") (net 28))
 (segment (start 61.722 58.166) (end 70.358 58.166) (width 0.3) (layer "B.Cu") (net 28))
 (segment (start 72.898 73.406) (end 68.58 73.406) (width 0.3) (layer "B.Cu") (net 28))
 (segment (start 73.406 61.214) (end 73.406 72.898) (width 0.3) (layer "B.Cu") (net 28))
 (segment (start 75.184 75.692) (end 72.898 73.406) (width 0.3) (layer "B.Cu") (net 28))
 (segment (start 70.358 58.166) (end 73.406 61.214) (width 0.3) (layer "B.Cu") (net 28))
 (segment (start 68.58 83.566) (end 72.39 83.566) (width 0.3) (layer "B.Cu") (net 24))
 (segment (start 68.58 81.026) (end 72.39 81.026) (width 0.3) (layer "B.Cu") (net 25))
 (segment (start 36.566 91.196) (end 36.576 91.186) (width 0.8) (layer "B.Cu") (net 33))
 (segment (start 33.02 91.196) (end 36.566 91.196) (width 0.8) (layer "B.Cu") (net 33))
 (segment (start 33.02 88.656) (end 36.566 88.656) (width 0.8) (layer "B.Cu") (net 34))
 (segment (start 36.566 88.656) (end 36.576 88.646) (width 0.8) (layer "B.Cu") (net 34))
 (segment (start 36.566 93.736) (end 36.576 93.726) (width 0.8) (layer "B.Cu") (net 32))
 (segment (start 33.02 93.736) (end 36.566 93.736) (width 0.8) (layer "B.Cu") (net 32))
 (segment (start 36.566 96.276) (end 36.576 96.266) (width 0.8) (layer "B.Cu") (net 31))
 (segment (start 33.02 96.276) (end 36.566 96.276) (width 0.8) (layer "B.Cu") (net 31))
 (segment (start 49.276 98.806) (end 53.34 98.806) (width 0.3) (layer "B.Cu") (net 15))
 (segment (start 49.276 83.566) (end 53.34 83.566) (width 0.3) (layer "B.Cu") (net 9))
 (segment (start 53.34 96.266) (end 49.276 96.266) (width 0.25) (layer "B.Cu") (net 14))
 (segment (start 49.276 93.726) (end 53.34 93.726) (width 0.25) (layer "B.Cu") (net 13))
 (segment (start 49.276 86.106) (end 53.34 86.106) (width 0.25) (layer "B.Cu") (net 10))
 (segment (start 49.276 88.646) (end 53.34 88.646) (width 0.25) (layer "B.Cu") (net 11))
 (segment (start 54.102 58.166) (end 54.102 55.118) (width 0.25) (layer "B.Cu") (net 2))
 (segment (start 49.53 58.166) (end 54.102 58.166) (width 0.25) (layer "B.Cu") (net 2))
 (segment (start 54.102 55.118) (end 52.832 53.848) (width 0.25) (layer "B.Cu") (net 2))
 (segment (start 56.642 66.802) (end 55.118 68.326) (width 0.3) (layer "B.Cu") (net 3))
 (segment (start 55.118 68.326) (end 53.34 68.326) (width 0.3) (layer "B.Cu") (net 3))
 (segment (start 56.642 58.166) (end 56.642 66.802) (width 0.3) (layer "B.Cu") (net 3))
 (segment (start 53.34 65.786) (end 49.53 65.786) (width 0.25) (layer "B.Cu") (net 1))
 (segment (start 68.58 65.786) (end 67.056 65.786) (width 0.25) (layer "B.Cu") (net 30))
 (segment (start 67.056 65.786) (end 60.706 72.136) (width 0.25) (layer "B.Cu") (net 30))
 (segment (start 39.37 98.806) (end 36.576 98.806) (width 0.25) (layer "B.Cu") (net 30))
 (segment (start 57.912 104.902) (end 46.26 104.902) (width 0.25) (layer "B.Cu") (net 30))
 (segment (start 60.706 102.108) (end 57.912 104.902) (width 0.25) (layer "B.Cu") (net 30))
 (segment (start 40.68 100.116) (end 39.37 98.806) (width 0.25) (layer "B.Cu") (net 30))
 (segment (start 40.68 110.482) (end 40.68 100.116) (width 0.25) (layer "B.Cu") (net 30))
 (segment (start 60.706 72.136) (end 60.706 102.108) (width 0.25) (layer "B.Cu") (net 30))
 (segment (start 46.26 104.902) (end 40.68 110.482) (width 0.25) (layer "B.Cu") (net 30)))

